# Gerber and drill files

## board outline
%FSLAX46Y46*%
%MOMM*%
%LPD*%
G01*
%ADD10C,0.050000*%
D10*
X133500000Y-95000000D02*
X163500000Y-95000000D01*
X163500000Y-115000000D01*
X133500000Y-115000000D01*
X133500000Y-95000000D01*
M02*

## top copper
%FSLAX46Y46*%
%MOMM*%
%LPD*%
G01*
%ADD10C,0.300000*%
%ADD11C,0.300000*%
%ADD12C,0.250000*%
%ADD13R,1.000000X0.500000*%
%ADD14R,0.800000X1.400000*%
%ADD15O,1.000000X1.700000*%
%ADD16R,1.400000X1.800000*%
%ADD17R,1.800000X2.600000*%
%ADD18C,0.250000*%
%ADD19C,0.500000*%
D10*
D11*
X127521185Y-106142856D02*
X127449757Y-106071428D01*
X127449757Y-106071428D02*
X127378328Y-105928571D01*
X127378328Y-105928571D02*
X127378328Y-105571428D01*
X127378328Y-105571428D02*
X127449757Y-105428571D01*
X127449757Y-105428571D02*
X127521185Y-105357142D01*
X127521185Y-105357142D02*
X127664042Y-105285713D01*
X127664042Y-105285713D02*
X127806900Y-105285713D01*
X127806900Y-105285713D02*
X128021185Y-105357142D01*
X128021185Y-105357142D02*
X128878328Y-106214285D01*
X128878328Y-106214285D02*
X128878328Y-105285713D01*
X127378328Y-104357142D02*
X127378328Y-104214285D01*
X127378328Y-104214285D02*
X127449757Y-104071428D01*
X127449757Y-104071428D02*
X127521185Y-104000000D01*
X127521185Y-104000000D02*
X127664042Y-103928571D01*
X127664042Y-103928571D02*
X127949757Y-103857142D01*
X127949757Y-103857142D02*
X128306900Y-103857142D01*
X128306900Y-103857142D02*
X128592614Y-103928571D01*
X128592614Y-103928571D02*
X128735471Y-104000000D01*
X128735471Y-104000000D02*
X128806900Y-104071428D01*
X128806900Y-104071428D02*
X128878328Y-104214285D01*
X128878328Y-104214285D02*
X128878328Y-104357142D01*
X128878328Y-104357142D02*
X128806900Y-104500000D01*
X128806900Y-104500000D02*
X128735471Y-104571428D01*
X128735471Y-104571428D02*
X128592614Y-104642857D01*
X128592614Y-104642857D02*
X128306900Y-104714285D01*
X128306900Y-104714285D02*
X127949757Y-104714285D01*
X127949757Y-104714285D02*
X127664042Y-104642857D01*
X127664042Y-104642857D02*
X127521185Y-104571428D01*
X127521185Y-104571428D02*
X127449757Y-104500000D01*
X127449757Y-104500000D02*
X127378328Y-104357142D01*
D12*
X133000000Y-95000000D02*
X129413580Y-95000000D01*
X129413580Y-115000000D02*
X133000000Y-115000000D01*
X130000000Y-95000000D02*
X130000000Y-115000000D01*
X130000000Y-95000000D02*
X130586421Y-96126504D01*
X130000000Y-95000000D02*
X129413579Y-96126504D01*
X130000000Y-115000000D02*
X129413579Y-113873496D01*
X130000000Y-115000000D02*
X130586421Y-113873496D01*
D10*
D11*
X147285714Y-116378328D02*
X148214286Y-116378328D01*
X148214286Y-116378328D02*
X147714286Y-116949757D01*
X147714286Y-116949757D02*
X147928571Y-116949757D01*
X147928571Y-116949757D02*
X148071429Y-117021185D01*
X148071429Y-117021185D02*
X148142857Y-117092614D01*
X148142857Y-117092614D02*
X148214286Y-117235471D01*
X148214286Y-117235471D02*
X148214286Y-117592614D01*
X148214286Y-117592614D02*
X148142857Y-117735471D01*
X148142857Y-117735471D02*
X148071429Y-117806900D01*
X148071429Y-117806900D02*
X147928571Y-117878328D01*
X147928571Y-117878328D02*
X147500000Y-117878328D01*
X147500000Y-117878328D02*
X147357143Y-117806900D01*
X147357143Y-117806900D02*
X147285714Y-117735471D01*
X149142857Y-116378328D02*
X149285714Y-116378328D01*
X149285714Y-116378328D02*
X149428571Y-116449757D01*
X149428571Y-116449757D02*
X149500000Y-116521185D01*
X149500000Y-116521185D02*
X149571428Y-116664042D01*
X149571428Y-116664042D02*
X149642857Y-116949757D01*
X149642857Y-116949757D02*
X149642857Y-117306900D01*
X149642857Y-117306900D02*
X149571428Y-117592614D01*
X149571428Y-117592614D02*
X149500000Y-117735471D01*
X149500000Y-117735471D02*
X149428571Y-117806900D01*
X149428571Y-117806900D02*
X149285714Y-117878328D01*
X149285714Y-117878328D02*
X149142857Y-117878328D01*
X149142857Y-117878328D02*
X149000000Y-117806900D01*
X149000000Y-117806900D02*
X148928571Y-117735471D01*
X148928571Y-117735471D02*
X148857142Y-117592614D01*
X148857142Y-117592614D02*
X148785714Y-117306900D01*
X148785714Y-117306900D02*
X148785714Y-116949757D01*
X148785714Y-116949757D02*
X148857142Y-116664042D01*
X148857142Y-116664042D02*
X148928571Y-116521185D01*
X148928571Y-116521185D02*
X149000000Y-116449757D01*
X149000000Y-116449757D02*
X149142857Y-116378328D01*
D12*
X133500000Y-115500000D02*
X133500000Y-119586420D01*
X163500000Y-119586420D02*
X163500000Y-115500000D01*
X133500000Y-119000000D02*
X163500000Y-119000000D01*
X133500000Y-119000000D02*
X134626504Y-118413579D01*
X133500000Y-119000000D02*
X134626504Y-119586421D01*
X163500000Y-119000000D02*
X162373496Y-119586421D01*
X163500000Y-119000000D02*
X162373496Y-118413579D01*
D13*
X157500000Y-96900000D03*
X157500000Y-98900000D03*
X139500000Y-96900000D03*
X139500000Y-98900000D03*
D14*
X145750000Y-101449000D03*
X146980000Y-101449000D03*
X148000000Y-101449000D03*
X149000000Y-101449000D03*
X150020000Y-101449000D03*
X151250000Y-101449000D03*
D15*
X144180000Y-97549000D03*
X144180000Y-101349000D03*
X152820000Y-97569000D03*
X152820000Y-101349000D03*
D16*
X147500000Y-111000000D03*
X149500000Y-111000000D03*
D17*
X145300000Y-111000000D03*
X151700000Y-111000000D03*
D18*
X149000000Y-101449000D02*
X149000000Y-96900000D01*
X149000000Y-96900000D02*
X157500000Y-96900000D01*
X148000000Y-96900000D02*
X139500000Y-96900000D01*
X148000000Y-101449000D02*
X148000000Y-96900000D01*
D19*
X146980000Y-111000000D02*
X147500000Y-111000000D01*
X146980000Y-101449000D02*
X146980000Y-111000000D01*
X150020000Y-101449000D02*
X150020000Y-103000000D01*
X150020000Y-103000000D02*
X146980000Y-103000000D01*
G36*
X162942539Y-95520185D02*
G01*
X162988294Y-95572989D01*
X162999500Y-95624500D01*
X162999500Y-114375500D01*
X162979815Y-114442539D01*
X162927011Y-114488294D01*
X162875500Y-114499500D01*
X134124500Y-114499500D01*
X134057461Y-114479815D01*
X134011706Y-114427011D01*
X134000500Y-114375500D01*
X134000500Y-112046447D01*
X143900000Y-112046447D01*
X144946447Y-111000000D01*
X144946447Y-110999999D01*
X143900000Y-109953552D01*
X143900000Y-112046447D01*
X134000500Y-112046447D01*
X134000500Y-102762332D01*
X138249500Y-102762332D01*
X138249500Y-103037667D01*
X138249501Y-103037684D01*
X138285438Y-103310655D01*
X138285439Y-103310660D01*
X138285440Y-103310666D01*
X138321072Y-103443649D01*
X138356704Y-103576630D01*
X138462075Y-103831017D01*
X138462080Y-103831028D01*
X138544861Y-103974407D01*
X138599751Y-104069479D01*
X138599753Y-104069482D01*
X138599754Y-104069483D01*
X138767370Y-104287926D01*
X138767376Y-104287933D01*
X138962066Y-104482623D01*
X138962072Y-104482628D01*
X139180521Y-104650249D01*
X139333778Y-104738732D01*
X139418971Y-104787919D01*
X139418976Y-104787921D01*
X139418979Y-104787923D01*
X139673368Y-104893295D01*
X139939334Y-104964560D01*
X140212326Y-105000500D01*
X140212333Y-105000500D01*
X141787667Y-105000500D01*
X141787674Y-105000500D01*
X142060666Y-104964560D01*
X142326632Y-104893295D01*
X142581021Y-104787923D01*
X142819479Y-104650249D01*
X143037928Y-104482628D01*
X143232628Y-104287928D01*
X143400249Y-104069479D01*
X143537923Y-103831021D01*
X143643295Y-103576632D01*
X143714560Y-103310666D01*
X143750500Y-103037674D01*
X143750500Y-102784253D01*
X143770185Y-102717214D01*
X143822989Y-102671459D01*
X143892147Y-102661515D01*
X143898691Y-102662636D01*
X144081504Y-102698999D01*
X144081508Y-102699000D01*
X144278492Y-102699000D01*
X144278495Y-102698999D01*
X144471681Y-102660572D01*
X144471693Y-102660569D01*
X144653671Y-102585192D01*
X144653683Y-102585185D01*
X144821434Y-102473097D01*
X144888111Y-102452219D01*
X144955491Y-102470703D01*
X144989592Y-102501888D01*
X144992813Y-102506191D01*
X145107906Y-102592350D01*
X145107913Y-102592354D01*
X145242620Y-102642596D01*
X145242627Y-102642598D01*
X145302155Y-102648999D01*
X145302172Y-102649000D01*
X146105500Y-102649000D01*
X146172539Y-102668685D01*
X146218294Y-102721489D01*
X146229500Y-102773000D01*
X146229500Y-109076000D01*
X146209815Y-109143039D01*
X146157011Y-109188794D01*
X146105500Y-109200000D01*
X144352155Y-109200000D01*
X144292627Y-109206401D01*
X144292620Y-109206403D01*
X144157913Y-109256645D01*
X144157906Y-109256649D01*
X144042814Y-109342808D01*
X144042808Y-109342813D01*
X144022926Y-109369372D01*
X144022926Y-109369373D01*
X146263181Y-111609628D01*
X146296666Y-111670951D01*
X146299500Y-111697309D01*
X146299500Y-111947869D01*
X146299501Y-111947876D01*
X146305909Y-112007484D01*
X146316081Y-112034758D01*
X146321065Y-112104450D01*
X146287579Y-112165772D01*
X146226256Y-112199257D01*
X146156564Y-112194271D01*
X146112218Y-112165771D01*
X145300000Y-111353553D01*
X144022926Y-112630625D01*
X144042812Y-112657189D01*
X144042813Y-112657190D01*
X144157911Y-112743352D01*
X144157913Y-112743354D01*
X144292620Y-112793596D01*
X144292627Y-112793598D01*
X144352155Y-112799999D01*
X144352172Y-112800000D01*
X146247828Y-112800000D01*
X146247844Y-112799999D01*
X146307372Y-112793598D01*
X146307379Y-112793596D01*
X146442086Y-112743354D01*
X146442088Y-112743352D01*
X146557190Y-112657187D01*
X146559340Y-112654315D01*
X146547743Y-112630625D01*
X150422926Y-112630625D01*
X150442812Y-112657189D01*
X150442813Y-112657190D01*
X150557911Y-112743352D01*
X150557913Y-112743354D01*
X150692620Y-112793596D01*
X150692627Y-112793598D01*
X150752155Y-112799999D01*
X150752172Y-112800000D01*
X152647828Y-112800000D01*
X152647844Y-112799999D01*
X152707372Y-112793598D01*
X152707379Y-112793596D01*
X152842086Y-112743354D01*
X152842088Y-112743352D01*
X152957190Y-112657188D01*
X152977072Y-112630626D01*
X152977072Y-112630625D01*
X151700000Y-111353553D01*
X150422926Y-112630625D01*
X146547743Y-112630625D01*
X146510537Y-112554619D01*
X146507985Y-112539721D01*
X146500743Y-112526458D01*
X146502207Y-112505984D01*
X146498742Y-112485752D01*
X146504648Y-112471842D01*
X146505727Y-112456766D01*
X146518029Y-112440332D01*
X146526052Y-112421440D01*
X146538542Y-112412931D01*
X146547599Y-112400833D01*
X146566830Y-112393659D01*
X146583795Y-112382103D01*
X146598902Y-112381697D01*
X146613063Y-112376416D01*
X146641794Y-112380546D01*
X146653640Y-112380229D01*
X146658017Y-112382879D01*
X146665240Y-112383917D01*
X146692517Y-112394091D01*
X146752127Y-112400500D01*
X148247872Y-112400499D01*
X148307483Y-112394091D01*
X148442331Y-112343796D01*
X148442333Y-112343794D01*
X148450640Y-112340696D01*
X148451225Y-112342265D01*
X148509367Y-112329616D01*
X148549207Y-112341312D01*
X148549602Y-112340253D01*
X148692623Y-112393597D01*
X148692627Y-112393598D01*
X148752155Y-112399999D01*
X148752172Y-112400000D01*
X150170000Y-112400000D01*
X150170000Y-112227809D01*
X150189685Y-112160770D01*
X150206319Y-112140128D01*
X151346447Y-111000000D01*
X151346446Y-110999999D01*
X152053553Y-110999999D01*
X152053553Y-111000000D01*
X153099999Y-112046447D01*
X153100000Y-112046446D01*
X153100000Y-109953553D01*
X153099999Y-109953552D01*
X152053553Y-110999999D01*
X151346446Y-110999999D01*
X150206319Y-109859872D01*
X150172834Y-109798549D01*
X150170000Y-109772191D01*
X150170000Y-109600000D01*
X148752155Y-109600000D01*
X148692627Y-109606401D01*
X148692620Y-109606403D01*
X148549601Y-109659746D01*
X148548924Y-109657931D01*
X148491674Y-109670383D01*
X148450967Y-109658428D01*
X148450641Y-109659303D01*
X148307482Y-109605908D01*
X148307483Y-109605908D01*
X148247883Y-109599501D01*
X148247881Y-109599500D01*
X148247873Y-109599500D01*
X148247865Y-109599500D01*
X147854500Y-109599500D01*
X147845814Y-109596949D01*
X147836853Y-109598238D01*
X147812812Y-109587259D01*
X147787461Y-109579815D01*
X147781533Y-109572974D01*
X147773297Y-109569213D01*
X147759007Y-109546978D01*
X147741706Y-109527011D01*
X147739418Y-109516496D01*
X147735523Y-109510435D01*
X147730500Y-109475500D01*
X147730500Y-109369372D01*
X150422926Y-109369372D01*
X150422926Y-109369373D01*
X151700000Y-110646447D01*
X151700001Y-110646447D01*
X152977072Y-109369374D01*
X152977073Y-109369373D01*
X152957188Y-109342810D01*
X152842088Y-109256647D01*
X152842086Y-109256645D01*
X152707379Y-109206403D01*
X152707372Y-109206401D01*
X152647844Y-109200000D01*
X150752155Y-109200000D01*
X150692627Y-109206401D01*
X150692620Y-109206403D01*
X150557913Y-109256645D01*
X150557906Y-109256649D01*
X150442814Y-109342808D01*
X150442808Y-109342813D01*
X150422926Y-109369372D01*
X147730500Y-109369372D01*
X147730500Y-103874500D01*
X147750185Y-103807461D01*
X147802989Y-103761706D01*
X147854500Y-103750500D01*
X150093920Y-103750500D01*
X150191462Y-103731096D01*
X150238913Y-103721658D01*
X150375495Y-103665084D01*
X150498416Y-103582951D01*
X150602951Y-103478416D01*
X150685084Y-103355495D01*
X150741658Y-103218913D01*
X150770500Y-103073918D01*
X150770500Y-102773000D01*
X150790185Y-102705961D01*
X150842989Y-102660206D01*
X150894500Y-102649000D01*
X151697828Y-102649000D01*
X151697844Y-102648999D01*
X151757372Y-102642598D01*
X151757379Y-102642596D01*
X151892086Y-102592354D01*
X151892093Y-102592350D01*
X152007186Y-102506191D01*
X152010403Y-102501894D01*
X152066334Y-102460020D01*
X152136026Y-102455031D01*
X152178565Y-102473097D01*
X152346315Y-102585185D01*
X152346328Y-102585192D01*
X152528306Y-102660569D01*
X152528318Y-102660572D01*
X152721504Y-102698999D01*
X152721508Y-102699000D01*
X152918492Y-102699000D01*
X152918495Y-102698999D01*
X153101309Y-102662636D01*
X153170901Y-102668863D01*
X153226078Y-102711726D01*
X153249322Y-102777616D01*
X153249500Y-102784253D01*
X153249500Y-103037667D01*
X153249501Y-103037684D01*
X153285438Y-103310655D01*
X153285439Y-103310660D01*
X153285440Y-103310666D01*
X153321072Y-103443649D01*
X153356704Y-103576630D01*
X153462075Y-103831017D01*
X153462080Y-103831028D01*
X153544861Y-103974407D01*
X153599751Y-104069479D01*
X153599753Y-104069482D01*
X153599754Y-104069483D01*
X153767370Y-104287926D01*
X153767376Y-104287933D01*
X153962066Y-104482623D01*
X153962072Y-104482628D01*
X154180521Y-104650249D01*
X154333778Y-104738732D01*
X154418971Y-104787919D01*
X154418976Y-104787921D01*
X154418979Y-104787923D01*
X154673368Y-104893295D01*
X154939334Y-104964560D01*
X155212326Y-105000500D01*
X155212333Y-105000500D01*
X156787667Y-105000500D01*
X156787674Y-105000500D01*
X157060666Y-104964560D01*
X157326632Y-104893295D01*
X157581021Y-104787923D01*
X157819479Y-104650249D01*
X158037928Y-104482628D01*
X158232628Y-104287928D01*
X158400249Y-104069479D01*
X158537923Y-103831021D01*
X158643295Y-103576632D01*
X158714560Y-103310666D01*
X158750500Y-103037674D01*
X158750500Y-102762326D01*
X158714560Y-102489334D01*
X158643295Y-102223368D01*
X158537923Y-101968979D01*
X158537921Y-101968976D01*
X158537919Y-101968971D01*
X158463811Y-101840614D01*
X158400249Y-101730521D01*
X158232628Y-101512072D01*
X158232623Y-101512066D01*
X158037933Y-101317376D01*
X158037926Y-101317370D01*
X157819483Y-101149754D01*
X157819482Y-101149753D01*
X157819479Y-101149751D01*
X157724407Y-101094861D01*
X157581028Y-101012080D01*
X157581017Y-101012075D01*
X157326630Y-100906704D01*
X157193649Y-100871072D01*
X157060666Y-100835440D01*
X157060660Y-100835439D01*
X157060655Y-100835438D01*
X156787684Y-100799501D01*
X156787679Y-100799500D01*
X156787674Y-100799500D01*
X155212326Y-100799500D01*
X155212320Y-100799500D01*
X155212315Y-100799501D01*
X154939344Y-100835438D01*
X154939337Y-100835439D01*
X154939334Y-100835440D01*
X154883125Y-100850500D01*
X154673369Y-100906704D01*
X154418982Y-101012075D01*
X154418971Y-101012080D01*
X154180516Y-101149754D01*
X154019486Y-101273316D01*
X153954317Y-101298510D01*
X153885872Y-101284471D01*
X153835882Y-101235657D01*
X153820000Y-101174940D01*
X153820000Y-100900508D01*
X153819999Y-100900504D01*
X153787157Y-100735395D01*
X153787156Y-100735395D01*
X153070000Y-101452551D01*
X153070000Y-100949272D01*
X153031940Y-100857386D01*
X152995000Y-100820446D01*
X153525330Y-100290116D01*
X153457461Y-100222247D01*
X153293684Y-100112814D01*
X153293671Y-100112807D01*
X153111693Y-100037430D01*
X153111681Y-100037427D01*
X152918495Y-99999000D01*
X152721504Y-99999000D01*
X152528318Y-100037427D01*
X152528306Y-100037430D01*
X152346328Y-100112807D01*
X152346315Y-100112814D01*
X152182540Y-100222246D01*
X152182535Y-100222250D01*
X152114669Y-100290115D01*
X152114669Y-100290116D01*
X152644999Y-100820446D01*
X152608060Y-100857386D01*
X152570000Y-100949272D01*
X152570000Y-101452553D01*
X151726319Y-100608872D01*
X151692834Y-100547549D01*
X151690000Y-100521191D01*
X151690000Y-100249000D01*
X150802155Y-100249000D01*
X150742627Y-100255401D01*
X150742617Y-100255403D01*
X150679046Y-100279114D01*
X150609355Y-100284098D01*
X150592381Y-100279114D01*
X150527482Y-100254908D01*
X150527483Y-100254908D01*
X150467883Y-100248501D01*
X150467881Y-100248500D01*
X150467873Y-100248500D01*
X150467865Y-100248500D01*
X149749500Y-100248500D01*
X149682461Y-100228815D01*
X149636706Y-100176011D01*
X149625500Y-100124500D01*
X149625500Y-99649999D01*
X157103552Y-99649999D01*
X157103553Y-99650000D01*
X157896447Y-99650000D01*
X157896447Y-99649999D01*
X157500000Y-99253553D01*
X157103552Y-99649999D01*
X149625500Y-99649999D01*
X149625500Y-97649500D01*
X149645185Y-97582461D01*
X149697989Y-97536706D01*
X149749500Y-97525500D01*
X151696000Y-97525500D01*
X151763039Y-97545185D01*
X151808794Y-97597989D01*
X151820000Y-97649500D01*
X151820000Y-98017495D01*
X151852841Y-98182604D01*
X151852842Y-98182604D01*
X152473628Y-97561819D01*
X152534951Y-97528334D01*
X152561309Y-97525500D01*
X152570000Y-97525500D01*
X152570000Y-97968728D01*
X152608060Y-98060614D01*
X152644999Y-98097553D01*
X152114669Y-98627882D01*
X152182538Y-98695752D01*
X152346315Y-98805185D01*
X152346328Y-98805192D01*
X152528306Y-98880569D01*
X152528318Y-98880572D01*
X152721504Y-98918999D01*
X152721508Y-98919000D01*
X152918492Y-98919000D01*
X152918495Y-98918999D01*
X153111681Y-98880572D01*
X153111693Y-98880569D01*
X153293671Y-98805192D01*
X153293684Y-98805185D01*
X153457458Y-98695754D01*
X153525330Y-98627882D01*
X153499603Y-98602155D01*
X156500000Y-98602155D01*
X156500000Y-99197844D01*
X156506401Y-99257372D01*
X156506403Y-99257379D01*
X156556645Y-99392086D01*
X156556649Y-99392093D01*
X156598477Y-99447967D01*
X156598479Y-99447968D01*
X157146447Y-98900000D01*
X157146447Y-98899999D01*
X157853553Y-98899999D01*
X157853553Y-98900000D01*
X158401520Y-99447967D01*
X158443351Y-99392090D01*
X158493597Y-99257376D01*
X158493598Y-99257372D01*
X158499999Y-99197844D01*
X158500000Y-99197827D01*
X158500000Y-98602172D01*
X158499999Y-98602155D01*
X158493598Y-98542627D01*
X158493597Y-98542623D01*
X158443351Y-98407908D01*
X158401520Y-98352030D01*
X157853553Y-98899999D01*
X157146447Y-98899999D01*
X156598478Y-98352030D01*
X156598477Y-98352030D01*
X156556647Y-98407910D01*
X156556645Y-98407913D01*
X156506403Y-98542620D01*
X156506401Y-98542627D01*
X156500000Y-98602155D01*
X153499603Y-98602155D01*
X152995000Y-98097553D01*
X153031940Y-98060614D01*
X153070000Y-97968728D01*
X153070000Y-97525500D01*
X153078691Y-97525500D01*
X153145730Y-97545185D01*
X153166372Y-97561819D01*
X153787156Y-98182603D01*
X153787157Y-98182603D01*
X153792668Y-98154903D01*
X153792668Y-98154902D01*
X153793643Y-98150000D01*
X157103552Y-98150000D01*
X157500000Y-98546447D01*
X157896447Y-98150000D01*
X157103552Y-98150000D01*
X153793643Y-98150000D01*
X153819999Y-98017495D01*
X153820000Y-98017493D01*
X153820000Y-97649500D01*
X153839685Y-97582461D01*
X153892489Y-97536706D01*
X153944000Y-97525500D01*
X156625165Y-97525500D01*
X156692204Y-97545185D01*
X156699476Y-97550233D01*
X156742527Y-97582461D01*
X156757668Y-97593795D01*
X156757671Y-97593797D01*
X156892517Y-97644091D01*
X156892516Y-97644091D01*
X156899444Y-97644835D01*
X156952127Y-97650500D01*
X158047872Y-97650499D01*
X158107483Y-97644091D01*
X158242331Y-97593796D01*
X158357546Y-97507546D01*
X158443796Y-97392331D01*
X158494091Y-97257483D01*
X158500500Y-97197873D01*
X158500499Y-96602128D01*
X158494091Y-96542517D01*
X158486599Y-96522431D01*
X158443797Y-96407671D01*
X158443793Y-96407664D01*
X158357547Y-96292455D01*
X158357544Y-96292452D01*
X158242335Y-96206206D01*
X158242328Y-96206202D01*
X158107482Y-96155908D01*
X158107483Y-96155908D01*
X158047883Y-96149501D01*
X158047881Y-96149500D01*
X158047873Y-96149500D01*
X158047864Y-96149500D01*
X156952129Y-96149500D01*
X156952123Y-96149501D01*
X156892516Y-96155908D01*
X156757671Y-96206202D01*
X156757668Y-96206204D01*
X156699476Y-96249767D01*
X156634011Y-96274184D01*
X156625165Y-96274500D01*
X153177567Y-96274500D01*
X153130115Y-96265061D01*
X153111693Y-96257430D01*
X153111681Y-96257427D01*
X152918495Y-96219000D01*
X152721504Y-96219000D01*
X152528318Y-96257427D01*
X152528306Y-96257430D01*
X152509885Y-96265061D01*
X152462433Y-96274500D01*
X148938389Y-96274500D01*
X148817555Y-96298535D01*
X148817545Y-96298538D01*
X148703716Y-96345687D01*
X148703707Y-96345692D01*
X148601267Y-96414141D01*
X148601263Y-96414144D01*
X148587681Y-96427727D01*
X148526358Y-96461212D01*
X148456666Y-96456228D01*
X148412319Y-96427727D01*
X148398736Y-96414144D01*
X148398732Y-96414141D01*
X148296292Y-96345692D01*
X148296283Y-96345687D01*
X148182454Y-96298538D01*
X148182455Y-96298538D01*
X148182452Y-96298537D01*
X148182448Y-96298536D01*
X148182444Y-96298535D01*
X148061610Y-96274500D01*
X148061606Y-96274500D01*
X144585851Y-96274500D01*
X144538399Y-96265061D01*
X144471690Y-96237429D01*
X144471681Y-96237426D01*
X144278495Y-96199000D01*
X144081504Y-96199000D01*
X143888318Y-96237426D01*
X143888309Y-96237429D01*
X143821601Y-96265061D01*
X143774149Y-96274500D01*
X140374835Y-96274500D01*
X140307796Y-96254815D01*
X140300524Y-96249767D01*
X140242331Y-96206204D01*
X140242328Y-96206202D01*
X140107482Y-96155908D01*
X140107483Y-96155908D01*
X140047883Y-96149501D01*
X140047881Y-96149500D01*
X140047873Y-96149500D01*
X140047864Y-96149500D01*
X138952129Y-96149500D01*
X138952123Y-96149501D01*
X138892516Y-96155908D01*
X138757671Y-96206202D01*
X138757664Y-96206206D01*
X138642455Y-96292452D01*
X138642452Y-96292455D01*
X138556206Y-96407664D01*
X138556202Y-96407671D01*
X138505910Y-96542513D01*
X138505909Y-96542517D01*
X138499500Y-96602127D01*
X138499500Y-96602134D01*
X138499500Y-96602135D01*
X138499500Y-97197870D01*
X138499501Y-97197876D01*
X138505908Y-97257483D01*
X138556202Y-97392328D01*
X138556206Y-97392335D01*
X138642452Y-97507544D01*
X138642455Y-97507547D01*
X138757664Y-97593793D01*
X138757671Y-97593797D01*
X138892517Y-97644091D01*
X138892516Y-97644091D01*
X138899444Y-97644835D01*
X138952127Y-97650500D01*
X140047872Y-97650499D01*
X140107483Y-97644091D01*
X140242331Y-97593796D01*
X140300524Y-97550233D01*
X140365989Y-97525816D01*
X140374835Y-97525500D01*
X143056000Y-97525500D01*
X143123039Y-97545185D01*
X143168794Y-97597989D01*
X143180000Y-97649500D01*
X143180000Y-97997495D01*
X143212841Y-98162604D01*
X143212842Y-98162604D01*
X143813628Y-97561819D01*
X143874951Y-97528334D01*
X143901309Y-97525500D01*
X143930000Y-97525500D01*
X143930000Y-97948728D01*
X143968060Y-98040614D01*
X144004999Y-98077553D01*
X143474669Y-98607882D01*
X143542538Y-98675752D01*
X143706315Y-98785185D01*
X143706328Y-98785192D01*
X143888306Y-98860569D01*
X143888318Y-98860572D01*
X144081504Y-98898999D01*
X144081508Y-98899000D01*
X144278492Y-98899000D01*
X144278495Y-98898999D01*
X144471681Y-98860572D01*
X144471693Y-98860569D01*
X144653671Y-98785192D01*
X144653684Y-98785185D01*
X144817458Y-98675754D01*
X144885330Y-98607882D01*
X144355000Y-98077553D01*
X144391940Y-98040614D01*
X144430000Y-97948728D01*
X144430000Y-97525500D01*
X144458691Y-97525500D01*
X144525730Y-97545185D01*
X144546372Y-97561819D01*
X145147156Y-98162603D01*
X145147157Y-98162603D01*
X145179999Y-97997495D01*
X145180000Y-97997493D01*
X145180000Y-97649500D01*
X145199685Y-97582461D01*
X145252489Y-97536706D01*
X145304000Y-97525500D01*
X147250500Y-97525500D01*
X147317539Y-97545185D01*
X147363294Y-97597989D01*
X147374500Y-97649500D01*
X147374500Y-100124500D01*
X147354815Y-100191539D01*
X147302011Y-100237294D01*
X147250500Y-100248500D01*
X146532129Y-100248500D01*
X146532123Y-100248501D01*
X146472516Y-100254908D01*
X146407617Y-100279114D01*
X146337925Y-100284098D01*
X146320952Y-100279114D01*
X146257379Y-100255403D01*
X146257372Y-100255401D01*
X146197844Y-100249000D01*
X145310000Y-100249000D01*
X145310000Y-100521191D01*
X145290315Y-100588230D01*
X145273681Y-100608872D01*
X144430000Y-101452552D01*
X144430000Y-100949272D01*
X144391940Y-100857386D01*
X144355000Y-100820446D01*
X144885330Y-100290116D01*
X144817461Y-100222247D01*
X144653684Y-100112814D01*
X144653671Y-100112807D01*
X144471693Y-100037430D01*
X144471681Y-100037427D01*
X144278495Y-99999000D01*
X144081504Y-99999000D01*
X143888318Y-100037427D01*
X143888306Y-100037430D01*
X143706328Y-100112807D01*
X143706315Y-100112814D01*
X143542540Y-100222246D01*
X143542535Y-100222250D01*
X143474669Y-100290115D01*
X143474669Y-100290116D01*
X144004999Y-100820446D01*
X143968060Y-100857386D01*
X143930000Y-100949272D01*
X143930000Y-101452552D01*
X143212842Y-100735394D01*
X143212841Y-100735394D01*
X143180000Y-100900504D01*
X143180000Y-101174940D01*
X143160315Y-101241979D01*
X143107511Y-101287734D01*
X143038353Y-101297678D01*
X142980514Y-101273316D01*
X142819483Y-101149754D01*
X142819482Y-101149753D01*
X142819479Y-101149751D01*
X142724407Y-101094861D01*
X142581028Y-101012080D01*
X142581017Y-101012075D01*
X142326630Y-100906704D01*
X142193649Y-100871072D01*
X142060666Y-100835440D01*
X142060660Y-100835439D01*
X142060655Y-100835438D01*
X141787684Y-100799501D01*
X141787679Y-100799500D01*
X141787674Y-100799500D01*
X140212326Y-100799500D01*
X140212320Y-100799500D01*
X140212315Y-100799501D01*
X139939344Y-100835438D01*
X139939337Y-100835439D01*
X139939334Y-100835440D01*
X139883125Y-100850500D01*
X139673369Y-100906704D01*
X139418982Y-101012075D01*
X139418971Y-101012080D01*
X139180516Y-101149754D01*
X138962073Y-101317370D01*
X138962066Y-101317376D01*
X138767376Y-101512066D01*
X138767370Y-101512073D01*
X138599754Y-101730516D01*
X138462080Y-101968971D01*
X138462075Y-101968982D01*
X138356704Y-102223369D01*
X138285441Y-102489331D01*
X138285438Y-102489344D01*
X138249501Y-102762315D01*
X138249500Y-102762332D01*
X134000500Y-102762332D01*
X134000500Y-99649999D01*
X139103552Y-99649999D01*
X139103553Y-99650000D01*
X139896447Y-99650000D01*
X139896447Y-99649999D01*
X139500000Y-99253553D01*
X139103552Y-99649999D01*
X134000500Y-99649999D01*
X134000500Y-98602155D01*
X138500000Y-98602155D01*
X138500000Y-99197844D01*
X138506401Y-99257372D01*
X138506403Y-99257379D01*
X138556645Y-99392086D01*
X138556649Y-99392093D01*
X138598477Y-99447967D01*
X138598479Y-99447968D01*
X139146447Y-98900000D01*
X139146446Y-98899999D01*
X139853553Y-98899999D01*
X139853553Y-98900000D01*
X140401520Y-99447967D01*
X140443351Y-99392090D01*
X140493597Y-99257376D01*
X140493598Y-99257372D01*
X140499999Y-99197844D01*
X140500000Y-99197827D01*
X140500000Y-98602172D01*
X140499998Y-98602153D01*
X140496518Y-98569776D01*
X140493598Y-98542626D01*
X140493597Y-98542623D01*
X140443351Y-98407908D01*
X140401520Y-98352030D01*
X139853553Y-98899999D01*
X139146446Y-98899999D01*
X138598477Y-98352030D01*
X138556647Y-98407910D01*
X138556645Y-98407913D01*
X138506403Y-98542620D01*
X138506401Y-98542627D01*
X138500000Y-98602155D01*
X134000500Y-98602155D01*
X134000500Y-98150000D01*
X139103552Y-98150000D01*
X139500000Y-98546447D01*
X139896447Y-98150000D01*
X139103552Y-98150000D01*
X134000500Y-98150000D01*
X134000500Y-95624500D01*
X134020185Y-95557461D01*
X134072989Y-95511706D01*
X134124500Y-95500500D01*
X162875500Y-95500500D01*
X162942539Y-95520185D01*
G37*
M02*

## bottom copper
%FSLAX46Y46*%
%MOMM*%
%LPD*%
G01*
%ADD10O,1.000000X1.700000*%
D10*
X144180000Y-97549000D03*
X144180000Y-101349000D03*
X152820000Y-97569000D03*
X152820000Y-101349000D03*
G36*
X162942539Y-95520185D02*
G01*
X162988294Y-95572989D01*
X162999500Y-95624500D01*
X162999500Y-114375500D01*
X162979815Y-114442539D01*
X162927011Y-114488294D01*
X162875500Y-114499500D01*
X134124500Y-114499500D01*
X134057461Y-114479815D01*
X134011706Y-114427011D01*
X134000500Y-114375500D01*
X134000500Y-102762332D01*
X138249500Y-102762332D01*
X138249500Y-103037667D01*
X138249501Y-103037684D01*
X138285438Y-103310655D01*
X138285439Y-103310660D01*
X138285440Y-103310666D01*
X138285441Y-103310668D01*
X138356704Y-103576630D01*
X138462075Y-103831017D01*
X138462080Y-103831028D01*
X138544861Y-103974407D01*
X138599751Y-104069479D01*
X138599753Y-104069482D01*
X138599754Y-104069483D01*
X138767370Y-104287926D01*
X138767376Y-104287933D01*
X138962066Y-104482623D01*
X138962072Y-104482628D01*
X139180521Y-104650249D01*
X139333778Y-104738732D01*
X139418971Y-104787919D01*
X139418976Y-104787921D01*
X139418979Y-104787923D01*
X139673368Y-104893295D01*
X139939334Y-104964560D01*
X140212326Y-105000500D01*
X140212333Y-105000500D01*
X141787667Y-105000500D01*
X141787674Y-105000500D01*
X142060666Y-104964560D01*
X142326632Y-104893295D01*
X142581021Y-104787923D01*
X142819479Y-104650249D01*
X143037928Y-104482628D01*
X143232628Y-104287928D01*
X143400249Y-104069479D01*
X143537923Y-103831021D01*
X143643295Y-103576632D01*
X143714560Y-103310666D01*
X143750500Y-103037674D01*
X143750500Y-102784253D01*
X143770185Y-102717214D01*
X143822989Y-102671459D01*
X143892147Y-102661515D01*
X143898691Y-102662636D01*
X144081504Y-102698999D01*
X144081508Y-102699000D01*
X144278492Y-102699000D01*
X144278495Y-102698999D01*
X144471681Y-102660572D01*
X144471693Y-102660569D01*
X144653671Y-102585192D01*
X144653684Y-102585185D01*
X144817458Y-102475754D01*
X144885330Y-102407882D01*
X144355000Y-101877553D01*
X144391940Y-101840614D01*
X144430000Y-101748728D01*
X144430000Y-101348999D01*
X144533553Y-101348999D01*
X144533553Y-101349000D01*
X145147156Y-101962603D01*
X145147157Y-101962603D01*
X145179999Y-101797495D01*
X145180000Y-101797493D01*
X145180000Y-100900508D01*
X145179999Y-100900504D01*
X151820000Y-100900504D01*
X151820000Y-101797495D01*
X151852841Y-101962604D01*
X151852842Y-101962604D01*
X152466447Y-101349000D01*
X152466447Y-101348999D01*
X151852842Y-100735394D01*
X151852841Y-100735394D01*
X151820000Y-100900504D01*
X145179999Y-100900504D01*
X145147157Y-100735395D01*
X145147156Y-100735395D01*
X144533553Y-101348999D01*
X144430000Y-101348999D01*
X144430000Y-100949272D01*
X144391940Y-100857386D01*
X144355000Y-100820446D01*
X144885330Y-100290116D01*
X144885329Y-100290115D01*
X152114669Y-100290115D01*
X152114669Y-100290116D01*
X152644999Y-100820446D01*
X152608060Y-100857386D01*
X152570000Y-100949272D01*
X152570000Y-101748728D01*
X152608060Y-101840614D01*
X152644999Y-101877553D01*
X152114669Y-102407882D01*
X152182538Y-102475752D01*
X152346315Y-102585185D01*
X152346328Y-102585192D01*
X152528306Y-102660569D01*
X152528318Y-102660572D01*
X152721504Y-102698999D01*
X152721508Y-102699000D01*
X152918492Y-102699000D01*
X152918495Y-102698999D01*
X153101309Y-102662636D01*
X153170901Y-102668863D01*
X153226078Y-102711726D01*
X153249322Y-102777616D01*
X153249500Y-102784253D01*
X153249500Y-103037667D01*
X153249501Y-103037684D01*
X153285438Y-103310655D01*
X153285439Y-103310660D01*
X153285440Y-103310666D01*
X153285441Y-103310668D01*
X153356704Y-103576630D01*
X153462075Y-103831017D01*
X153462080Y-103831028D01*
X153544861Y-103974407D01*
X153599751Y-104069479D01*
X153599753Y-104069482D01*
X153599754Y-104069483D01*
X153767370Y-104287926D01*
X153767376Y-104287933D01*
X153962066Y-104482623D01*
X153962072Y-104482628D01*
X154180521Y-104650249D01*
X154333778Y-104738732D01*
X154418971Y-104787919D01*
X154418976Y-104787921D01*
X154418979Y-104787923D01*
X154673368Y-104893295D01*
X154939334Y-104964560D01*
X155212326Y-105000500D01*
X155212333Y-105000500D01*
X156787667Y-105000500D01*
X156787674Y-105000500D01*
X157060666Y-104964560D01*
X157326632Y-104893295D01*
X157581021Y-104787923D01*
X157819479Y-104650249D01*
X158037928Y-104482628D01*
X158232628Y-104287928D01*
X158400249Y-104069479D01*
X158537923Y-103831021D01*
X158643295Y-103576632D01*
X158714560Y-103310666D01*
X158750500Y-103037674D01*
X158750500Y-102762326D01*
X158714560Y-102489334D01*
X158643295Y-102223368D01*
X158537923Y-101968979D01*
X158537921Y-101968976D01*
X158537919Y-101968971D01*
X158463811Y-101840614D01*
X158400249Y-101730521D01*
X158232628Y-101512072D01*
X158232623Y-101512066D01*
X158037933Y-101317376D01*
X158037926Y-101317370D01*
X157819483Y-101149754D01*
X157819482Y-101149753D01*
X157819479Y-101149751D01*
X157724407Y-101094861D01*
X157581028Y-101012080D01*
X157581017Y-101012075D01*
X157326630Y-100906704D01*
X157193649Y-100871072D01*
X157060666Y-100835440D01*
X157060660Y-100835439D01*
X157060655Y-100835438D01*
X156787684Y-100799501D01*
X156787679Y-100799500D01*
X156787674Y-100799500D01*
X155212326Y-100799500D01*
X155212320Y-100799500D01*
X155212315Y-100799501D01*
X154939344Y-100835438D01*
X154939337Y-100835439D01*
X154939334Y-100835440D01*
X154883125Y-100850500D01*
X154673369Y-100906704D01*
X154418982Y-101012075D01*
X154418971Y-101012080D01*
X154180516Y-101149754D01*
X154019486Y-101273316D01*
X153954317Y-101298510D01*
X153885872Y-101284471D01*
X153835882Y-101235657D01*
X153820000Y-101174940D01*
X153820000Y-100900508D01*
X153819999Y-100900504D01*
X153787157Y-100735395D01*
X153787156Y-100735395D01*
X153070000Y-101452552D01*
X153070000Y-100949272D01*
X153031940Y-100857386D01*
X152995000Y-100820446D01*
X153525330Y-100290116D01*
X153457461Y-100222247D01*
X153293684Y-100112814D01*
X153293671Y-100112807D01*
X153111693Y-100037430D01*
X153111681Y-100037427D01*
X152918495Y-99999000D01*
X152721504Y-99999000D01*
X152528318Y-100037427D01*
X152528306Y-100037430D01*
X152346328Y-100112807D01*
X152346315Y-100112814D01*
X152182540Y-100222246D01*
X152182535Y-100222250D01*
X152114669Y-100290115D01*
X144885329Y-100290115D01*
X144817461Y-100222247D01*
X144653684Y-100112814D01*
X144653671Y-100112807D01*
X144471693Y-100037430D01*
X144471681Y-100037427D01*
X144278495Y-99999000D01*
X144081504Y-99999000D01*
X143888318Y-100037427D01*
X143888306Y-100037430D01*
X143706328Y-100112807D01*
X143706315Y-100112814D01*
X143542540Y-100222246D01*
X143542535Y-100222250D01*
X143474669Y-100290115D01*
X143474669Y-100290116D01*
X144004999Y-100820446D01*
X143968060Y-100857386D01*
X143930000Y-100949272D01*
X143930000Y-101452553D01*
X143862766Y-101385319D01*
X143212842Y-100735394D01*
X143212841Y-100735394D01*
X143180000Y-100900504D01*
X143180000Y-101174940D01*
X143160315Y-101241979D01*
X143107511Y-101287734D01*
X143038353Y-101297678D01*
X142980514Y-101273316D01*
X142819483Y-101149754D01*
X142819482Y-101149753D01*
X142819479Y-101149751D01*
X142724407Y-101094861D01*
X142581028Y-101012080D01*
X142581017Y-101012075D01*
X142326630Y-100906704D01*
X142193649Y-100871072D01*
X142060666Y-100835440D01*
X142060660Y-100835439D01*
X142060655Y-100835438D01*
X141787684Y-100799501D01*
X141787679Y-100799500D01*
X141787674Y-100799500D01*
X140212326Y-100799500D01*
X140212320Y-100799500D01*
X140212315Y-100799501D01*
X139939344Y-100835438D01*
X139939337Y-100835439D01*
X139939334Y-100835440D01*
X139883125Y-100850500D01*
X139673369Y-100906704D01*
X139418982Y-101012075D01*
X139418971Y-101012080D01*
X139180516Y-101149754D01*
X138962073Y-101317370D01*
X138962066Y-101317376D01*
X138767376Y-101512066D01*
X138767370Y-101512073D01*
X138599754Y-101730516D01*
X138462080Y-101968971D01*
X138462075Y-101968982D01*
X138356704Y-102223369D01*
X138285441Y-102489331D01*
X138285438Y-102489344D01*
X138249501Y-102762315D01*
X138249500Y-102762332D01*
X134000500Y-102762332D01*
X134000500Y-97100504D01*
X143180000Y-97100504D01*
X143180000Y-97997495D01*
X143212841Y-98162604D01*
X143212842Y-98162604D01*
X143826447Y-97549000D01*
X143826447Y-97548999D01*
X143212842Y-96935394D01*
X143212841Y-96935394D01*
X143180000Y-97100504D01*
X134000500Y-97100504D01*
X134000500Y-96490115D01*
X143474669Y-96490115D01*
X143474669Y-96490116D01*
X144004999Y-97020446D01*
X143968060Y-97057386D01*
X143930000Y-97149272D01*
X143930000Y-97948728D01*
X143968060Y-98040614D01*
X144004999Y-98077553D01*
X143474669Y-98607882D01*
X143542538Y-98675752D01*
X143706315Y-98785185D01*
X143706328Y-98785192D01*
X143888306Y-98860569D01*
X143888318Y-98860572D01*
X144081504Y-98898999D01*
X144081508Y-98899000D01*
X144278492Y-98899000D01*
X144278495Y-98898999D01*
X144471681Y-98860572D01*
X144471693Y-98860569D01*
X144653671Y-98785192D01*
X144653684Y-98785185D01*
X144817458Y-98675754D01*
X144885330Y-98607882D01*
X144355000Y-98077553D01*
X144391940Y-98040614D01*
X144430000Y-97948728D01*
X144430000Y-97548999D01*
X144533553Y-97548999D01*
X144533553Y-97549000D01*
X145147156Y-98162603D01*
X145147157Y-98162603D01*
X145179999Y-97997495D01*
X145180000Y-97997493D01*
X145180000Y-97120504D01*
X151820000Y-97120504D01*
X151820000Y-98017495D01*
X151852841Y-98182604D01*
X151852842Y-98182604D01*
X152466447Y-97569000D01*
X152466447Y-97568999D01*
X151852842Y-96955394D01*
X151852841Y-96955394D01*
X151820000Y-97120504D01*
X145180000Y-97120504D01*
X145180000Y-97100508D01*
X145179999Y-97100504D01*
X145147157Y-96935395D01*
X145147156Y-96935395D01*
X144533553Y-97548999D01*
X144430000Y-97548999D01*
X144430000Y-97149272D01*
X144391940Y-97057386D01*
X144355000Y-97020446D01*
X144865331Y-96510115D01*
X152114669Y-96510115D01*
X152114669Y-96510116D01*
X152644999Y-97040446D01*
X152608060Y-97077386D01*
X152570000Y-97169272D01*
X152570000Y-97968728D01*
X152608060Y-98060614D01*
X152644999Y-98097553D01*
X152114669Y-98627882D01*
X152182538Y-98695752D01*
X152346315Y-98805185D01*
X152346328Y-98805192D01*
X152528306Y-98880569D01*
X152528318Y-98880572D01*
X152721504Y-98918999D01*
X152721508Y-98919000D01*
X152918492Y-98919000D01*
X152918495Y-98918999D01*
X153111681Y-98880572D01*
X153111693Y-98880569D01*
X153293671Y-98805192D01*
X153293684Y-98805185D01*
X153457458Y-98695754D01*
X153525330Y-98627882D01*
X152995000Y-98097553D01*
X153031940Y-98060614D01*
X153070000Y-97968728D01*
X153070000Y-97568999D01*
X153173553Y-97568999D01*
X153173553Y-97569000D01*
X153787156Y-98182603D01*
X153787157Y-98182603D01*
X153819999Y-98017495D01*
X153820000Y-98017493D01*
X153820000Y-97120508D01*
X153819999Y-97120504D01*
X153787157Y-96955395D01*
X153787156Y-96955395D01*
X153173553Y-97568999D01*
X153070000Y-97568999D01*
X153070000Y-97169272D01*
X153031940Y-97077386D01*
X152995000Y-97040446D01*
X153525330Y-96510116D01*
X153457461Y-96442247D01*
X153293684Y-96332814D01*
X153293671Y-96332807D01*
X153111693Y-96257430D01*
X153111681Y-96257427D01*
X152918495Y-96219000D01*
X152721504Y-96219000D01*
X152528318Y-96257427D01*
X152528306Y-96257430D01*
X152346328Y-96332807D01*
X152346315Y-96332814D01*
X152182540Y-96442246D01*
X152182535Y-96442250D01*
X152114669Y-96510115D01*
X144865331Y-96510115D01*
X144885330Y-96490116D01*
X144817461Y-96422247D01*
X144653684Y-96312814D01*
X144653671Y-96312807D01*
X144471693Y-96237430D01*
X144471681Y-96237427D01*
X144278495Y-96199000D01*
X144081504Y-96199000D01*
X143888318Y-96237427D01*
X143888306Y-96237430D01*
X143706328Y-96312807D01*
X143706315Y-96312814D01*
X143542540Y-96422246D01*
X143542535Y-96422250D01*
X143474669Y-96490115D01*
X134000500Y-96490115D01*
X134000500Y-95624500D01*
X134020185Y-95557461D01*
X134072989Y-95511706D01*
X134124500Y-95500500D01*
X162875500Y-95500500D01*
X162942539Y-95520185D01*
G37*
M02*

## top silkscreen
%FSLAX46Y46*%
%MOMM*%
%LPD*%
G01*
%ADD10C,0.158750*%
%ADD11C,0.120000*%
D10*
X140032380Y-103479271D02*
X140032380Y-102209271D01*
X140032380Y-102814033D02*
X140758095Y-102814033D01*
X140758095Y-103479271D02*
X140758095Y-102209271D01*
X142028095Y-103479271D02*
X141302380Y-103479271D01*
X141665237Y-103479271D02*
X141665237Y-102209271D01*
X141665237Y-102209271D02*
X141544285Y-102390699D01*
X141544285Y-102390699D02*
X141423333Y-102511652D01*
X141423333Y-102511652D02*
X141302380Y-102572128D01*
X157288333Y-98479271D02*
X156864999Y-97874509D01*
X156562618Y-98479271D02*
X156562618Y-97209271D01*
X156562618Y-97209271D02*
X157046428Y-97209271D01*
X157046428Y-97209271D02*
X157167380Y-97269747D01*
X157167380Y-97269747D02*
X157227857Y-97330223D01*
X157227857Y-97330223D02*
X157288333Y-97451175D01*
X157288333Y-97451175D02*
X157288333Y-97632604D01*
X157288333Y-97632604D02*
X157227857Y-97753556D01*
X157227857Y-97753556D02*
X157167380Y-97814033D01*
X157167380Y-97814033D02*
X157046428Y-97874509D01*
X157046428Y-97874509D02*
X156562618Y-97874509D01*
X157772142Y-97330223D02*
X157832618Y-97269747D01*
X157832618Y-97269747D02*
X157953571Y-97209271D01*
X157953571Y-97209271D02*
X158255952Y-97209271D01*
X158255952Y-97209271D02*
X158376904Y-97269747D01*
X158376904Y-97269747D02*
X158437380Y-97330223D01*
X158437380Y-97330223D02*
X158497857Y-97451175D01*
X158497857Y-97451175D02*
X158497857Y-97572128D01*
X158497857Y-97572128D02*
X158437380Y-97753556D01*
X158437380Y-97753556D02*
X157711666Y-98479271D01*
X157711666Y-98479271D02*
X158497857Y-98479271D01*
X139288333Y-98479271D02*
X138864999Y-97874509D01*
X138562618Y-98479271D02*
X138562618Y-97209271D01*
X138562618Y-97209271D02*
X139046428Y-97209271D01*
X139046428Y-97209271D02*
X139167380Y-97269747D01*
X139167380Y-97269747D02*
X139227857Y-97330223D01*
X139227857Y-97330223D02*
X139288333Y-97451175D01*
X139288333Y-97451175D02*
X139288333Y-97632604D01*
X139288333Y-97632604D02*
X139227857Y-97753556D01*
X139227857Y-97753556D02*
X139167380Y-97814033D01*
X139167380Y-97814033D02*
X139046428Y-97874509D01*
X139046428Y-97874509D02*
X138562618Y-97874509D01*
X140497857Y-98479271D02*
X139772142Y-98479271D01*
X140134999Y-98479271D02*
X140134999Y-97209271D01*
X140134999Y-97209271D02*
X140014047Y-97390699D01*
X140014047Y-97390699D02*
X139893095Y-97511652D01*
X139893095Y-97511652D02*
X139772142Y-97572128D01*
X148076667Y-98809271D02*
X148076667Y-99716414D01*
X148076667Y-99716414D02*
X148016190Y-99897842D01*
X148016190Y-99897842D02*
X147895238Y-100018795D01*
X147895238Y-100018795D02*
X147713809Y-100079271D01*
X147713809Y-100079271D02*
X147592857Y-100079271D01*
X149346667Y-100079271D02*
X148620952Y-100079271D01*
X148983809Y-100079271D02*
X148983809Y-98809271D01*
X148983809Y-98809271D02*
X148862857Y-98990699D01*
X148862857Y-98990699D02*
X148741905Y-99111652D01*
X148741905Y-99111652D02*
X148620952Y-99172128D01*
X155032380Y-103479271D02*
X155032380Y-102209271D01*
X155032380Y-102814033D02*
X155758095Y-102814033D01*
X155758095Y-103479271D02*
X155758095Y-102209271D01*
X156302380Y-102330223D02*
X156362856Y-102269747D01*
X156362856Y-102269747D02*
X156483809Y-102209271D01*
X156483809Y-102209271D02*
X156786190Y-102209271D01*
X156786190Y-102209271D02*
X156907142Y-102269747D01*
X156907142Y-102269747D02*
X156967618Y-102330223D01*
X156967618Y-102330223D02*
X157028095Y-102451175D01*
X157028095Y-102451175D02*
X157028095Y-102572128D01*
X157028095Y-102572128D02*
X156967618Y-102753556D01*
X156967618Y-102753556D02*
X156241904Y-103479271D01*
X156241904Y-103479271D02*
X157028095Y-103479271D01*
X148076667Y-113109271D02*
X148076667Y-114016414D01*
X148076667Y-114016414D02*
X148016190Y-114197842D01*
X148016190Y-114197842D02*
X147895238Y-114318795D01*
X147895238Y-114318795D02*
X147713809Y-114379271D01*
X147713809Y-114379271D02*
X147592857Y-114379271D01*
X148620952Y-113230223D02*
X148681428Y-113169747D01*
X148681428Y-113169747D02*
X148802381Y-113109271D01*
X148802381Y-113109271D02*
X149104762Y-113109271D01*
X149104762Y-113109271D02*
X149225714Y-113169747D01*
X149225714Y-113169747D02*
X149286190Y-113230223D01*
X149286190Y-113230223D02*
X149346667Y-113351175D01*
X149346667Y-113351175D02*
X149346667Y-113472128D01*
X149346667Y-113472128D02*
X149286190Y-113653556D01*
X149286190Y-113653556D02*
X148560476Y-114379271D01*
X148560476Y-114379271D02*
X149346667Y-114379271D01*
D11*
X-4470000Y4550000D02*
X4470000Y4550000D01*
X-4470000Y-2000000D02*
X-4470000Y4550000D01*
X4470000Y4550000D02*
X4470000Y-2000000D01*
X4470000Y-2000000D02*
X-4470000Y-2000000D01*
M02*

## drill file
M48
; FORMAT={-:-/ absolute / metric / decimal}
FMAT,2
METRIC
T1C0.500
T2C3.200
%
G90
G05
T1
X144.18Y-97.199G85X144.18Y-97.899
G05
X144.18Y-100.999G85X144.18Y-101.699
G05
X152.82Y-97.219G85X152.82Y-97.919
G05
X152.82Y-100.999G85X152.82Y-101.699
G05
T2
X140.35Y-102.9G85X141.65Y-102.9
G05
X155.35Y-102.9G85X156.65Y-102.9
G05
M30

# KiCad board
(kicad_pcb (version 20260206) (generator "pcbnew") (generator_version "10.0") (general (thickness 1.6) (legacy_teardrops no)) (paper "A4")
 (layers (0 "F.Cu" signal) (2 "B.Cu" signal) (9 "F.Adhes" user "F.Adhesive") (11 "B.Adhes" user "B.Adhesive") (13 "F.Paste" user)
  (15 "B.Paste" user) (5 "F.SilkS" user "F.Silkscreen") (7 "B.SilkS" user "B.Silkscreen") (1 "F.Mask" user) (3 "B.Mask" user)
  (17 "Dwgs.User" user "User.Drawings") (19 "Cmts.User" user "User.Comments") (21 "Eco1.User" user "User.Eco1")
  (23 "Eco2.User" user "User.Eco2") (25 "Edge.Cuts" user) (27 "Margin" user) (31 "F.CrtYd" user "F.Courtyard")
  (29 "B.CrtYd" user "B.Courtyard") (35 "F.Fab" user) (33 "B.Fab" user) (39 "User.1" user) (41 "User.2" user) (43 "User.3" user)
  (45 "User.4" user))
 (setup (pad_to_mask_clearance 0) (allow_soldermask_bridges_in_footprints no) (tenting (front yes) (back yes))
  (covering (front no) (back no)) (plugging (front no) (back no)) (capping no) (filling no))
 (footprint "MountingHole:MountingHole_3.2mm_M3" (layer "F.Cu") (at 141 102.9)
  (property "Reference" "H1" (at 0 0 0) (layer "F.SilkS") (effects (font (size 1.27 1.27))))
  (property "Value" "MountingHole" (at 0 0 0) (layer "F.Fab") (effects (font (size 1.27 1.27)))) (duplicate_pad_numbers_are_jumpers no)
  (pad "" np_thru_hole oval (at 0 0) (size 4.5 3.2) (drill oval 4.5 3.2) (layers "*.Cu")))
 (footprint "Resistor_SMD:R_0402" (layer "F.Cu") (at 157.5 97.9)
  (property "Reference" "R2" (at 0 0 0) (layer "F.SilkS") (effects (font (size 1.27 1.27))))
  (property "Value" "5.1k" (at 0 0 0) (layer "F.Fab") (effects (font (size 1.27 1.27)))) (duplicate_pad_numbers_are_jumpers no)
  (pad "1" smd rect (at 0 -1) (size 1 0.5) (layers "F.Cu" "F.Mask" "F.Paste") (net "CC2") (thermal_bridge_angle 45))
  (pad "2" smd rect (at 0 1) (size 1 0.5) (layers "F.Cu" "F.Mask" "F.Paste") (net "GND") (thermal_bridge_angle 45)))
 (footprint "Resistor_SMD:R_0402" (layer "F.Cu") (at 139.5 97.9)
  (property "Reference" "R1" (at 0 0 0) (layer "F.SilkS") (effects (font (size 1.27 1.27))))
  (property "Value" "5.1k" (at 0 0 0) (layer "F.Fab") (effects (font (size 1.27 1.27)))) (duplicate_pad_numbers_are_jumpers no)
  (pad "1" smd rect (at 0 -1) (size 1 0.5) (layers "F.Cu" "F.Mask" "F.Paste") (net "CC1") (thermal_bridge_angle 45))
  (pad "2" smd rect (at 0 1) (size 1 0.5) (layers "F.Cu" "F.Mask" "F.Paste") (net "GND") (thermal_bridge_angle 45)))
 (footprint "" (layer "F.Cu") (at 148.5 99.5)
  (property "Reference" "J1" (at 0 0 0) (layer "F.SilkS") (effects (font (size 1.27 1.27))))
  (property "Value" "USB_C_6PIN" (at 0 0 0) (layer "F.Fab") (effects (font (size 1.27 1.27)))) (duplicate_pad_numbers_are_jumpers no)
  (fp_line (start -152.97 -104.05) (end -144.03 -104.05) (stroke (width 0.12) (type default)) (layer "F.SilkS"))
  (fp_line (start -152.97 -97.5) (end -152.97 -104.05) (stroke (width 0.12) (type default)) (layer "F.SilkS"))
  (fp_line (start -144.03 -104.05) (end -144.03 -97.5) (stroke (width 0.12) (type default)) (layer "F.SilkS"))
  (fp_line (start -144.03 -97.5) (end -152.97 -97.5) (stroke (width 0.12) (type default)) (layer "F.SilkS"))
  (pad "1" smd rect (at -2.75 1.949) (size 0.8 1.4) (layers "F.Cu" "F.Mask" "F.Paste") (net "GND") (thermal_bridge_angle 45))
  (pad "2" smd rect (at -1.52 1.949) (size 0.8 1.4) (layers "F.Cu" "F.Mask" "F.Paste") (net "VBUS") (thermal_bridge_angle 45))
  (pad "3" smd rect (at -0.5 1.949) (size 0.8 1.4) (layers "F.Cu" "F.Mask" "F.Paste") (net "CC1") (thermal_bridge_angle 45))
  (pad "4" smd rect (at 0.5 1.949) (size 0.8 1.4) (layers "F.Cu" "F.Mask" "F.Paste") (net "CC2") (thermal_bridge_angle 45))
  (pad "5" smd rect (at 1.52 1.949) (size 0.8 1.4) (layers "F.Cu" "F.Mask" "F.Paste") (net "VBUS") (thermal_bridge_angle 45))
  (pad "6" smd rect (at 2.75 1.949) (size 0.8 1.4) (layers "F.Cu" "F.Mask" "F.Paste") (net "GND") (thermal_bridge_angle 45))
  (pad "M1" thru_hole oval (at -4.32 -1.951) (size 1 1.7) (drill oval 0.5 1.2) (layers "*.Cu" "*.Mask") (remove_unused_layers no)
   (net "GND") (thermal_bridge_angle 45))
  (pad "M2" thru_hole oval (at -4.32 1.849) (size 1 1.7) (drill oval 0.5 1.2) (layers "*.Cu" "*.Mask") (remove_unused_layers no) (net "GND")
   (thermal_bridge_angle 45))
  (pad "M3" thru_hole oval (at 4.32 -1.931) (size 1 1.7) (drill oval 0.5 1.2) (layers "*.Cu" "*.Mask") (remove_unused_layers no) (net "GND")
   (thermal_bridge_angle 45))
  (pad "M4" thru_hole oval (at 4.32 1.849) (size 1 1.7) (drill oval 0.5 1.2) (layers "*.Cu" "*.Mask") (remove_unused_layers no) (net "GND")
   (thermal_bridge_angle 45)))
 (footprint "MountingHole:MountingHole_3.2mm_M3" (layer "F.Cu") (at 156 102.9)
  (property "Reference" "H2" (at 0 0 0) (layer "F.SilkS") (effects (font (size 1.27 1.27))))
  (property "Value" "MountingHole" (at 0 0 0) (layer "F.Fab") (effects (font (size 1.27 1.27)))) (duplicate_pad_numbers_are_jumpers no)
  (pad "" np_thru_hole oval (at 0 0) (size 4.5 3.2) (drill oval 4.5 3.2) (layers "*.Cu")))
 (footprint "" (layer "F.Cu") (at 148.5 111)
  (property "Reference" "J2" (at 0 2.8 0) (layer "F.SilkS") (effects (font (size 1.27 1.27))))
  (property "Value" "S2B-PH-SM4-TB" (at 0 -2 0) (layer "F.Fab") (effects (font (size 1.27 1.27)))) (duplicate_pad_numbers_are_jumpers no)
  (pad "1" smd rect (at -1 0) (size 1.4 1.8) (layers "F.Cu" "F.Mask" "F.Paste") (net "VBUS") (thermal_bridge_angle 45))
  (pad "2" smd rect (at 1 0) (size 1.4 1.8) (layers "F.Cu" "F.Mask" "F.Paste") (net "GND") (thermal_bridge_angle 45))
  (pad "MP1" smd rect (at -3.2 0) (size 1.8 2.6) (layers "F.Cu" "F.Mask" "F.Paste") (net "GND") (thermal_bridge_angle 45))
  (pad "MP2" smd rect (at 3.2 0) (size 1.8 2.6) (layers "F.Cu" "F.Mask" "F.Paste") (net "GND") (thermal_bridge_angle 45)))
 (gr_rect (start 133.5 95) (end 163.5 115) (stroke (width 0.05) (type default)) (fill no) (layer "Edge.Cuts"))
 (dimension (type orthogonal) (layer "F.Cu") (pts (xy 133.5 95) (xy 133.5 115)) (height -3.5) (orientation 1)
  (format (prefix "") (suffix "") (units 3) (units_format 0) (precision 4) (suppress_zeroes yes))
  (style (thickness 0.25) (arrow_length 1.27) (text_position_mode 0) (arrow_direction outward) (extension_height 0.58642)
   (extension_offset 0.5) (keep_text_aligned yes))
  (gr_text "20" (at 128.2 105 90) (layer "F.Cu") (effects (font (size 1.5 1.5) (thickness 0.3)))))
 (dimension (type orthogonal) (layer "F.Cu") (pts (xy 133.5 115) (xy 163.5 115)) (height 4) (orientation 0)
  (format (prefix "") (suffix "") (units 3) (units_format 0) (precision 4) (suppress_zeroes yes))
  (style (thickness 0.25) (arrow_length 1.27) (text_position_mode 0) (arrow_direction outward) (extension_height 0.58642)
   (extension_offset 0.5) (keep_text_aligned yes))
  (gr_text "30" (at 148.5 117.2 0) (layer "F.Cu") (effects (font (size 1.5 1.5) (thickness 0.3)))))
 (segment (start 149 101.449) (end 149 96.9) (width 0.25) (layer "F.Cu") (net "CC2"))
 (segment (start 149 96.9) (end 157.5 96.9) (width 0.25) (layer "F.Cu") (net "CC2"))
 (segment (start 148 96.9) (end 139.5 96.9) (width 0.25) (layer "F.Cu") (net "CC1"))
 (segment (start 148 101.449) (end 148 96.9) (width 0.25) (layer "F.Cu") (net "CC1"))
 (segment (start 146.98 111) (end 147.5 111) (width 0.5) (layer "F.Cu") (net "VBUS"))
 (segment (start 146.98 101.449) (end 146.98 111) (width 0.5) (layer "F.Cu") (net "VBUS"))
 (segment (start 150.02 101.449) (end 150.02 103) (width 0.5) (layer "F.Cu") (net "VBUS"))
 (segment (start 150.02 103) (end 146.98 103) (width 0.5) (layer "F.Cu") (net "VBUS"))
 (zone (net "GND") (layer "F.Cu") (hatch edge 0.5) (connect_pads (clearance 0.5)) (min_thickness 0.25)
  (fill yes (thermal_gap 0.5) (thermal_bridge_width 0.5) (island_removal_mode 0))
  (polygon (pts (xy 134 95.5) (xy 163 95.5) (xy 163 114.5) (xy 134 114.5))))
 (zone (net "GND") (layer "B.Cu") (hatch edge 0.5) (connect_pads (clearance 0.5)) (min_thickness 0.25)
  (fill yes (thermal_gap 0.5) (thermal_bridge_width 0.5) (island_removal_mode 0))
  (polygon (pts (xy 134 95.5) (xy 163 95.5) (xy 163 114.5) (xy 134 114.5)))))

